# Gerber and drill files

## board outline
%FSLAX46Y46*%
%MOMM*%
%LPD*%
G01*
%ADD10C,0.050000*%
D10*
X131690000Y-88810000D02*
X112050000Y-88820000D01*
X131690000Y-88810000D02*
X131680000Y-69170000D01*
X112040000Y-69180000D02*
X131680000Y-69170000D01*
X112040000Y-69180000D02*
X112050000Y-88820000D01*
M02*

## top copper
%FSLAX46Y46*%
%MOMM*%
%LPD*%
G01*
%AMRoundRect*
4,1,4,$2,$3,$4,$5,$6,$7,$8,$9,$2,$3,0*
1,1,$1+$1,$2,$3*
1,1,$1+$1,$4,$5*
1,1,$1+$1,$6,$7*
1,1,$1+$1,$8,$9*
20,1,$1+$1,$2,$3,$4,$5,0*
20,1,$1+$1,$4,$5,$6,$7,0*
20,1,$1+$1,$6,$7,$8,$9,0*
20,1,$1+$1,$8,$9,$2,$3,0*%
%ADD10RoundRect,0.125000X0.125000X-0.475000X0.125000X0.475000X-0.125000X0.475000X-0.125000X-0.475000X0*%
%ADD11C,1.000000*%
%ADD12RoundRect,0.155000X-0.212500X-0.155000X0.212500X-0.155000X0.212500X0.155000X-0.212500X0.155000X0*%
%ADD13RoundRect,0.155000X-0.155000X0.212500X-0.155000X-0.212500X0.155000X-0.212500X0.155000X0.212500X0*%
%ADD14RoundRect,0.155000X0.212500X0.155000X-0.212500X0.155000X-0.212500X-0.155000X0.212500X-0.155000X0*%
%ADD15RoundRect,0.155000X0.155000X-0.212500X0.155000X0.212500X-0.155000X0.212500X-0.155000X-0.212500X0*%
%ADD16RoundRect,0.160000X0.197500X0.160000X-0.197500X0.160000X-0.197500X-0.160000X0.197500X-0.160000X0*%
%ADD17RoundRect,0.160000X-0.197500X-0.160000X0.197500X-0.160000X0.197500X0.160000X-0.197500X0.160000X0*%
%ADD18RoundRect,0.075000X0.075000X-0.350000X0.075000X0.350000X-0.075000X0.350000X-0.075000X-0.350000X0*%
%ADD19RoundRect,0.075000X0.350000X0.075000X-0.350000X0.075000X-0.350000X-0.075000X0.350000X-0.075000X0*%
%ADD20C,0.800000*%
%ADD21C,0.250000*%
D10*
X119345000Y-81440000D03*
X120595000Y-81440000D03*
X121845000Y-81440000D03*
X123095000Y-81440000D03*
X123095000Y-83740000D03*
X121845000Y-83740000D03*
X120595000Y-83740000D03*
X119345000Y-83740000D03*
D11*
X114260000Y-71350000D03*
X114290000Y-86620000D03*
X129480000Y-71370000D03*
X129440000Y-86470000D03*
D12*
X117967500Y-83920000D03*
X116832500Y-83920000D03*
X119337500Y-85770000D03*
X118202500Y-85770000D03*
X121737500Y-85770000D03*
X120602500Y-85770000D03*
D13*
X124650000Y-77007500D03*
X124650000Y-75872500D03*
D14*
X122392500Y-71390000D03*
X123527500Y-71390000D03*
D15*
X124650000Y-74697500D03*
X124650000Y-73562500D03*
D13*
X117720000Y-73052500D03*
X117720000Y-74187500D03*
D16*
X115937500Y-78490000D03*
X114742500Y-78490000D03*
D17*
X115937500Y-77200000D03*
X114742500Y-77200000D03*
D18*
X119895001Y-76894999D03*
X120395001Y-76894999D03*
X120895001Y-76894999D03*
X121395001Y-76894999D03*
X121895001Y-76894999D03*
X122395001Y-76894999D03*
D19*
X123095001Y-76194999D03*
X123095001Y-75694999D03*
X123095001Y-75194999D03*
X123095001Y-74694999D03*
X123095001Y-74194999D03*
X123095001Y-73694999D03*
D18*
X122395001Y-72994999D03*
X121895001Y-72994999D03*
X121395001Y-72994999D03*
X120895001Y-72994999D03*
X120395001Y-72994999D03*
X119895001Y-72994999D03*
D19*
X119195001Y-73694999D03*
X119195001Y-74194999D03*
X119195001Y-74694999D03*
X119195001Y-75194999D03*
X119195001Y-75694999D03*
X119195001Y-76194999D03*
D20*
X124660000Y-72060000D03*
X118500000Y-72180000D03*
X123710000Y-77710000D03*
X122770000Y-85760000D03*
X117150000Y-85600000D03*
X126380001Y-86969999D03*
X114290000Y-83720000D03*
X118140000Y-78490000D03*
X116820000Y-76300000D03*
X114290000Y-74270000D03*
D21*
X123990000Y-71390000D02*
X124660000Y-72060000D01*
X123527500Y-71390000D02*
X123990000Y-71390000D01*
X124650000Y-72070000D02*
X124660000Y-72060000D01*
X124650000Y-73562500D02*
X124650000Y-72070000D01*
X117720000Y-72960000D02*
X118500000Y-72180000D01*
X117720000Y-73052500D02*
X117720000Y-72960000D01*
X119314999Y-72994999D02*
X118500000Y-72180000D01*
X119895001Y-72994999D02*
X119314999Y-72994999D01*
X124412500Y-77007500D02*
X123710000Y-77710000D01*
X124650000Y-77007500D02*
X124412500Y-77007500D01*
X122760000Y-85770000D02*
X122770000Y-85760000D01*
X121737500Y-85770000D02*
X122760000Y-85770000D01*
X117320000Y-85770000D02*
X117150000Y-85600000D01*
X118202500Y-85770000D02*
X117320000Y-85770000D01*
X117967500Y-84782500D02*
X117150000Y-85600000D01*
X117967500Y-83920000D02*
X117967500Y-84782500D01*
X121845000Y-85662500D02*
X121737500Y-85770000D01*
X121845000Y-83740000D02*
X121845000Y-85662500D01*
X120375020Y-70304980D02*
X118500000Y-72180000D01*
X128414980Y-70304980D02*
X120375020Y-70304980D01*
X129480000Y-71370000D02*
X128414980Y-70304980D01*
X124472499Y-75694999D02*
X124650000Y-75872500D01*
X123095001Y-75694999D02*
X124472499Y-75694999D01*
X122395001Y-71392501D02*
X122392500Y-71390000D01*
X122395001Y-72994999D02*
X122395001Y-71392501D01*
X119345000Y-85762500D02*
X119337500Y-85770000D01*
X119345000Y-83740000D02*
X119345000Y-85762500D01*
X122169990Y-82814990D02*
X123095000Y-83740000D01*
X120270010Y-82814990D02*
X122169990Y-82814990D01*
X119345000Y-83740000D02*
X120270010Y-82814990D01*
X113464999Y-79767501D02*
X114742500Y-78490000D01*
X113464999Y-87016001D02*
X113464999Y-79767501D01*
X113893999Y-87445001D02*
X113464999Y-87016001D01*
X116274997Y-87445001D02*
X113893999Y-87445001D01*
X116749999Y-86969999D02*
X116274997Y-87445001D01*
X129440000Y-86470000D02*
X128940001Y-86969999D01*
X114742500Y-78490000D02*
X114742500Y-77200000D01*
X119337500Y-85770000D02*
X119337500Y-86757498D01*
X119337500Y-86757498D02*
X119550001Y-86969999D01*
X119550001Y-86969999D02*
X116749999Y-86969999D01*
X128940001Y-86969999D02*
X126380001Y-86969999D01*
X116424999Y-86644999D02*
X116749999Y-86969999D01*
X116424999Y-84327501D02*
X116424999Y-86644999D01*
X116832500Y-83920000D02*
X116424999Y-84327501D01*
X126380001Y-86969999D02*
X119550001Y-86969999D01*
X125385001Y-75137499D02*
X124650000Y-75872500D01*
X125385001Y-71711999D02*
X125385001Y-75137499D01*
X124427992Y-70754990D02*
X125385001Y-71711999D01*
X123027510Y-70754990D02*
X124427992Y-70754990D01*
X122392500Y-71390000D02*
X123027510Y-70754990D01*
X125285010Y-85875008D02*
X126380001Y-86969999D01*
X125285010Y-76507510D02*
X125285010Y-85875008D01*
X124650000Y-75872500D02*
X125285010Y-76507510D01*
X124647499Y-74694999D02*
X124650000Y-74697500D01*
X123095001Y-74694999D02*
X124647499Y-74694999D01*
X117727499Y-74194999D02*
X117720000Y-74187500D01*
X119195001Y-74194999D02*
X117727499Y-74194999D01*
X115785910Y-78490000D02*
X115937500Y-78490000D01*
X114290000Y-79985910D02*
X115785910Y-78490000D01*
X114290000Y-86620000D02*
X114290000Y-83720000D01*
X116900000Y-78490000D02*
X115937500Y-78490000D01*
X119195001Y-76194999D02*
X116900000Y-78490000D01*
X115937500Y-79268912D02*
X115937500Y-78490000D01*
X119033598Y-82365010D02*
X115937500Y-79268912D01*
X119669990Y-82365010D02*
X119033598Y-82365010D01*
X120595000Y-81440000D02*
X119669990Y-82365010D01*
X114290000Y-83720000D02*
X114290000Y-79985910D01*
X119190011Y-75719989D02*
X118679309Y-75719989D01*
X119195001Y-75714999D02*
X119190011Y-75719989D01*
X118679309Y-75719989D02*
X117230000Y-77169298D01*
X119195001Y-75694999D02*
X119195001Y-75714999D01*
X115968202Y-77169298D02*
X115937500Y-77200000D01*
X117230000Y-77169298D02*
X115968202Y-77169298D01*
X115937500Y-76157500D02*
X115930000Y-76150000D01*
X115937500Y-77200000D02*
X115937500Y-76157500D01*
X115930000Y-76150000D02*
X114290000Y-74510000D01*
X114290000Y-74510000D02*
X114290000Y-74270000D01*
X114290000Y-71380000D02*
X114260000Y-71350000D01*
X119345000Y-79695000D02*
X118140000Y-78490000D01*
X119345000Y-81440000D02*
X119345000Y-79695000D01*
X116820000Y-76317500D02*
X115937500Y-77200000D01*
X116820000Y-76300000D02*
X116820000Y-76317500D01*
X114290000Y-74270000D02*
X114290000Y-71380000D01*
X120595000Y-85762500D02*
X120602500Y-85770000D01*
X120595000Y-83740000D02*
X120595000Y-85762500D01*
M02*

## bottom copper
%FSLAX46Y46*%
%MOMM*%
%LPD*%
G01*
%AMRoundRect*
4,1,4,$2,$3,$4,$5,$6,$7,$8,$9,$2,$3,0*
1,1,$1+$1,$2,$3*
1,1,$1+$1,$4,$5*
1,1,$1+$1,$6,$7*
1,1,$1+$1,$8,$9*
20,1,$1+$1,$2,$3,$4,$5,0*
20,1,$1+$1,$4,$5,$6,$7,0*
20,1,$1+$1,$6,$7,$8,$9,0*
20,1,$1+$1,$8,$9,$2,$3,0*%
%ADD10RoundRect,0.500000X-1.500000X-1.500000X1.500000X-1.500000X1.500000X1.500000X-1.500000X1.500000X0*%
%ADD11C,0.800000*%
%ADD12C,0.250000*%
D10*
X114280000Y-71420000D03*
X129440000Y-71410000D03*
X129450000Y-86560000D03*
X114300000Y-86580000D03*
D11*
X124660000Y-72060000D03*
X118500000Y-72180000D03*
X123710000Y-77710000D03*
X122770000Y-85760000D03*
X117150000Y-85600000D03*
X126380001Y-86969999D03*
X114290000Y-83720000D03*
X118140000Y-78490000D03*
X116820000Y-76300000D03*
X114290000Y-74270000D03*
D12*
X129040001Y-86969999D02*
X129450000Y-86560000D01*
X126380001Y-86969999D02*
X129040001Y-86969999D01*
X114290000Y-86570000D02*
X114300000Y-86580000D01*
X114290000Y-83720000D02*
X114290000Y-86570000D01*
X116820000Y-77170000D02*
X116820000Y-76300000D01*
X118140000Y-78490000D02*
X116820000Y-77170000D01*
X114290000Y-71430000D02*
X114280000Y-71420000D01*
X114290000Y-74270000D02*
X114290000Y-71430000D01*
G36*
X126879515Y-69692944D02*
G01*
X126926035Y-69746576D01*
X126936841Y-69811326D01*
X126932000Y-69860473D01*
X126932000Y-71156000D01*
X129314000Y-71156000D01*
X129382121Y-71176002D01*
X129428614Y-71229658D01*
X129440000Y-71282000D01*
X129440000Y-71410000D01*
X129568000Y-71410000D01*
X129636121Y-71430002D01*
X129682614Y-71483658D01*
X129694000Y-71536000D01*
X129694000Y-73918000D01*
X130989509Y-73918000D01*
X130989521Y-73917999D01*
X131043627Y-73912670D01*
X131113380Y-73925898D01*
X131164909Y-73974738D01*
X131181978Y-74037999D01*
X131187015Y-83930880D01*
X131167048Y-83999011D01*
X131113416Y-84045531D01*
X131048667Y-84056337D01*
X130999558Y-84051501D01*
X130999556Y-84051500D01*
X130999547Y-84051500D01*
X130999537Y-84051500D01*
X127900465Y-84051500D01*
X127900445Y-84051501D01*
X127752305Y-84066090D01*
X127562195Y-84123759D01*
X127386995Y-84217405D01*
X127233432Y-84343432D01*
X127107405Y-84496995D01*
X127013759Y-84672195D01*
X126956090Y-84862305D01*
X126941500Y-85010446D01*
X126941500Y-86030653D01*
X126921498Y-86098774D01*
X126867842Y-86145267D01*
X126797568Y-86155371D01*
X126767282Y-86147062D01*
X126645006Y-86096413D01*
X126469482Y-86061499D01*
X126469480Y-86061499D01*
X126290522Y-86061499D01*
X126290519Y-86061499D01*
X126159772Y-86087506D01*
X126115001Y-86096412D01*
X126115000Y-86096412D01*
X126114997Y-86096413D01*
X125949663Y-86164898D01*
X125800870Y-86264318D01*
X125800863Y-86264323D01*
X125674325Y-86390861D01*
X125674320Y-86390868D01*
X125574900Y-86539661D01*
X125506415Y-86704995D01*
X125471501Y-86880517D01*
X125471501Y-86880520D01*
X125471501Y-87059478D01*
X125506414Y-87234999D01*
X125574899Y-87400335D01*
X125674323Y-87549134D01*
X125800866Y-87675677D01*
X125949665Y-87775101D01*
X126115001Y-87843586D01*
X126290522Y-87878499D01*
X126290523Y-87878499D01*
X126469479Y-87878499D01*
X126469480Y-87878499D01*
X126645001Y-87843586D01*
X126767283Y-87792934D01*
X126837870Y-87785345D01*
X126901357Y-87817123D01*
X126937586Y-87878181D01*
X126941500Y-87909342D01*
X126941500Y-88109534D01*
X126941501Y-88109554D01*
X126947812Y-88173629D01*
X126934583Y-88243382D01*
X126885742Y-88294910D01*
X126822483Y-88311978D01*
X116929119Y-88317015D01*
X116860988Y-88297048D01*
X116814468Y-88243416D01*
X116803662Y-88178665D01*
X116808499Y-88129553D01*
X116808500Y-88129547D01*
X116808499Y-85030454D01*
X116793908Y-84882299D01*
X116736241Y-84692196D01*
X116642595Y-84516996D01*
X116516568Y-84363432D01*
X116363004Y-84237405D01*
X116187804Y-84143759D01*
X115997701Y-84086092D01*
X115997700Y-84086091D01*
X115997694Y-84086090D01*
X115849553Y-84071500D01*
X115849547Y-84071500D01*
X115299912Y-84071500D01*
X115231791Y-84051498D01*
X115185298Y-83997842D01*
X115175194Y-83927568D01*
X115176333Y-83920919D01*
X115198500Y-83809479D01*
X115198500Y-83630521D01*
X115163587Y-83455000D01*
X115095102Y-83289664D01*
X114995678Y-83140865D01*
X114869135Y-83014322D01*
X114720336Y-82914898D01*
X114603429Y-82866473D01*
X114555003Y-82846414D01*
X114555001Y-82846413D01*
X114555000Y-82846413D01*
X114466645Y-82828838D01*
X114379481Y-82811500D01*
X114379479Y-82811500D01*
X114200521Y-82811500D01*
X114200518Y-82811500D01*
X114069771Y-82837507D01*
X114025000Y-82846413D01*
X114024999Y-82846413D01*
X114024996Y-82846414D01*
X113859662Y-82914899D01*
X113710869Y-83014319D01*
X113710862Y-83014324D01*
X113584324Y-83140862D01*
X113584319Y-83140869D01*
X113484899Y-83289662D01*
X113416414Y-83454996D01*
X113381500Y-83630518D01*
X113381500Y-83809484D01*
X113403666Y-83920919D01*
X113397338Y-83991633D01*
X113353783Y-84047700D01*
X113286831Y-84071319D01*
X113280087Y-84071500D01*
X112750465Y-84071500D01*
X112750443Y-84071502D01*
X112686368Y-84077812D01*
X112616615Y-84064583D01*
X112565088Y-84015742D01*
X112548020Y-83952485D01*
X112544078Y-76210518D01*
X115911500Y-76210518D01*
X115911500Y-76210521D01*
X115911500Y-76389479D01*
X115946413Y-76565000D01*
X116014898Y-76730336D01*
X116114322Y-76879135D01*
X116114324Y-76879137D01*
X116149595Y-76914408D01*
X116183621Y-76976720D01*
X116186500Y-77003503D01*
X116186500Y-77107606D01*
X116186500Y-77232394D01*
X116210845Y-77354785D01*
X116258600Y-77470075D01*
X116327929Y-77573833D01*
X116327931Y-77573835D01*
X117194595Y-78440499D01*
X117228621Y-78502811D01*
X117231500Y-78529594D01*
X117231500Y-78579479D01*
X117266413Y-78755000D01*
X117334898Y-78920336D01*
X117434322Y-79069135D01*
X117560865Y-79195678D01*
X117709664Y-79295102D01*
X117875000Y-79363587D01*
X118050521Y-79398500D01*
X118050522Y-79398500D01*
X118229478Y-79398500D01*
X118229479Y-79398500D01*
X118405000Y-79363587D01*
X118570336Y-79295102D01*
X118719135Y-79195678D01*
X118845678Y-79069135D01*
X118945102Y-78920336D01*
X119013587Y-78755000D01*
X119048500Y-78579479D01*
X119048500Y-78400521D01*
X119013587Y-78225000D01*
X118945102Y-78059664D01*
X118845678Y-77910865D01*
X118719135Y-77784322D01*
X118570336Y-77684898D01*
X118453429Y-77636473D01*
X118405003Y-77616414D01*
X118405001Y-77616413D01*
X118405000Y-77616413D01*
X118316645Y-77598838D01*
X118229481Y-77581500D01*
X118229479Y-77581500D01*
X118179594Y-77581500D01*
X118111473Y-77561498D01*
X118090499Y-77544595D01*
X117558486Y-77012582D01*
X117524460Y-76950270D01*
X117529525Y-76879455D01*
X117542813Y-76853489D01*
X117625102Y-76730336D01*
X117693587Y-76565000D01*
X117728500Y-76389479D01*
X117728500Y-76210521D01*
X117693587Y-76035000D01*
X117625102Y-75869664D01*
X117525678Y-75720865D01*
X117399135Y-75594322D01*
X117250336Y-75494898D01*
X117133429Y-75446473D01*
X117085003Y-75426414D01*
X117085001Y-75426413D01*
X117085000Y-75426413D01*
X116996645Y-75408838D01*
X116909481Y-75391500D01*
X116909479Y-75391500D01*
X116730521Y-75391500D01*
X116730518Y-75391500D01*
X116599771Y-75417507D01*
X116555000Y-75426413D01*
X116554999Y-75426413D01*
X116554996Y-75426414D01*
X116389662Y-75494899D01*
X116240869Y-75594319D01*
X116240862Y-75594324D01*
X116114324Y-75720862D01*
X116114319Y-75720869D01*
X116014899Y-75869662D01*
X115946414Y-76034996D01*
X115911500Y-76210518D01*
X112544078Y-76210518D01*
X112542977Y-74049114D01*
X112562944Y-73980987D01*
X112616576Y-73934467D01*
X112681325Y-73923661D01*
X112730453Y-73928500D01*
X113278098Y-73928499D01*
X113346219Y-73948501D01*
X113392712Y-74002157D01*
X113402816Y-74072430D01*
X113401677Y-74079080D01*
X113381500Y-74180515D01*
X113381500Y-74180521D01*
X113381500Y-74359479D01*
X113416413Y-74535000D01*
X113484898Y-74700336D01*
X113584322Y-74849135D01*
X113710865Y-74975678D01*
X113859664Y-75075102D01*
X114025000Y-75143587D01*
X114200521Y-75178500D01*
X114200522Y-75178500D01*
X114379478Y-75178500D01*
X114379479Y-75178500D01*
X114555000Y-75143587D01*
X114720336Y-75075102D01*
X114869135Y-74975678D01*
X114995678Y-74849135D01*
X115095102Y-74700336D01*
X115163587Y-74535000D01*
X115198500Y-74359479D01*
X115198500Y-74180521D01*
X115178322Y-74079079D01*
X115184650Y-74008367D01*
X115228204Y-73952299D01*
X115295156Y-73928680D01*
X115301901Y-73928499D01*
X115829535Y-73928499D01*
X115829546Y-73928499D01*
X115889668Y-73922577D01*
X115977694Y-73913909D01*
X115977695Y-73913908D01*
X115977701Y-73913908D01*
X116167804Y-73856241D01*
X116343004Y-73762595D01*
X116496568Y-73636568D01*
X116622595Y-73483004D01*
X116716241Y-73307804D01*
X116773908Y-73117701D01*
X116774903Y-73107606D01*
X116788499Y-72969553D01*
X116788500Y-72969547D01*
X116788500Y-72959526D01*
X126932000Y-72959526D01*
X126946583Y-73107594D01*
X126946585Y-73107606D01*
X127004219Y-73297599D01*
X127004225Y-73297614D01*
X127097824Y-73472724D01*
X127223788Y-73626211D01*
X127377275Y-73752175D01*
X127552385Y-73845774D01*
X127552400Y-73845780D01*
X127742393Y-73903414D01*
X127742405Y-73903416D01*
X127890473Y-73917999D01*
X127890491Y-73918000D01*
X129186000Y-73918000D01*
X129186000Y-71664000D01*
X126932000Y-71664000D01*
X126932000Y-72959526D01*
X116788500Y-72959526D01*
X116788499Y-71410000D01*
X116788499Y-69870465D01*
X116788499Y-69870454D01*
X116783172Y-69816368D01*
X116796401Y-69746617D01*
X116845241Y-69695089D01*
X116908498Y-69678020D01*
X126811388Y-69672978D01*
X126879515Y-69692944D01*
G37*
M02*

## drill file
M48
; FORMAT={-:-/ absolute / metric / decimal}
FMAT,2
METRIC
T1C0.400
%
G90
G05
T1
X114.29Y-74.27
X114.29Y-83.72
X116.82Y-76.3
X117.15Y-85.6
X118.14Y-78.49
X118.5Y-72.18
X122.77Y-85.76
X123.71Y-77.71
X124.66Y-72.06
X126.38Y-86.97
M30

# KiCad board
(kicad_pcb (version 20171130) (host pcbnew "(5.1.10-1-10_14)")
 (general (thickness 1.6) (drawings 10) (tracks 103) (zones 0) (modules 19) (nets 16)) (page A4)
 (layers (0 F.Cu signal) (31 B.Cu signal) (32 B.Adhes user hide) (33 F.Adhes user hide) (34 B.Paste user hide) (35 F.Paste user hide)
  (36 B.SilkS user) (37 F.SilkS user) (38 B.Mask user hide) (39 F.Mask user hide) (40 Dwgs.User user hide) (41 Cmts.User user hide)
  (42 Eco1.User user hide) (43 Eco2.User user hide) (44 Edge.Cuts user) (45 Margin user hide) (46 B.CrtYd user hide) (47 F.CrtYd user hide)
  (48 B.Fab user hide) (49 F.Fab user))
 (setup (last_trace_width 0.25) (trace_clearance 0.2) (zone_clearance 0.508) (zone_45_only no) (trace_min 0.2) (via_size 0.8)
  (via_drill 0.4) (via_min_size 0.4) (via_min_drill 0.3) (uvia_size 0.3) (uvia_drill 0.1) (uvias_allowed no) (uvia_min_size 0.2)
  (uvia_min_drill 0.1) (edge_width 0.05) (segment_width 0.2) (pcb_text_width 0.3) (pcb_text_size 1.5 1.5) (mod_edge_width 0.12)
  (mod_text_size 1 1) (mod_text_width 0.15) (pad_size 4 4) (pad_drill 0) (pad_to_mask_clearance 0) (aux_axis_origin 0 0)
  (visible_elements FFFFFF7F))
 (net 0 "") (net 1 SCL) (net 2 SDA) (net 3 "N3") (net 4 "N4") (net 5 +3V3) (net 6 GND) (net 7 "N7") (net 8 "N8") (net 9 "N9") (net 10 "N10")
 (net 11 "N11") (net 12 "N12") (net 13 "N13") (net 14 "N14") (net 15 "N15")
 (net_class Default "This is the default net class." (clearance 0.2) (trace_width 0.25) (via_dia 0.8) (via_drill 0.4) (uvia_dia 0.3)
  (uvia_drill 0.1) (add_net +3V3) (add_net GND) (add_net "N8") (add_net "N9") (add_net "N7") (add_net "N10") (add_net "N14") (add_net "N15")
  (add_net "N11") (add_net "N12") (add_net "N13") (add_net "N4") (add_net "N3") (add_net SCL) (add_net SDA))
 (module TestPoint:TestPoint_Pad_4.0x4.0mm (layer B.Cu) (at 114.28 71.42)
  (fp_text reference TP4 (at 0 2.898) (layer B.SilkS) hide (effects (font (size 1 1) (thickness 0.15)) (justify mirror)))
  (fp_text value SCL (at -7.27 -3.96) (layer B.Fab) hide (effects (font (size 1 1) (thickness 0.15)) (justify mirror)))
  (pad 1 smd roundrect (at 0 0) (size 4 4) (layers B.Cu B.Paste B.Mask) (roundrect_rratio 0.125) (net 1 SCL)))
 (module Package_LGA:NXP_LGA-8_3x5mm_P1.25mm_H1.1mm (layer F.Cu) (at 121.22 82.59 90)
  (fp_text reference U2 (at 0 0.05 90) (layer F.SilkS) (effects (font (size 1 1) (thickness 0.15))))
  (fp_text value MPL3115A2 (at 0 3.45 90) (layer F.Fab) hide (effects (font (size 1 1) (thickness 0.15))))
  (pad 8 smd roundrect (at 1.15 -1.875 90) (size 1.2 0.5) (layers F.Cu F.Paste F.Mask) (roundrect_rratio 0.25) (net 1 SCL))
  (pad 7 smd roundrect (at 1.15 -0.625 90) (size 1.2 0.5) (layers F.Cu F.Paste F.Mask) (roundrect_rratio 0.25) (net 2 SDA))
  (pad 6 smd roundrect (at 1.15 0.625 90) (size 1.2 0.5) (layers F.Cu F.Paste F.Mask) (roundrect_rratio 0.25) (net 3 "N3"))
  (pad 5 smd roundrect (at 1.15 1.875 90) (size 1.2 0.5) (layers F.Cu F.Paste F.Mask) (roundrect_rratio 0.25) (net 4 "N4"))
  (pad 4 smd roundrect (at -1.15 1.875 90) (size 1.2 0.5) (layers F.Cu F.Paste F.Mask) (roundrect_rratio 0.25) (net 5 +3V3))
  (pad 3 smd roundrect (at -1.15 0.625 90) (size 1.2 0.5) (layers F.Cu F.Paste F.Mask) (roundrect_rratio 0.25) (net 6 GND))
  (pad 2 smd roundrect (at -1.15 -0.625 90) (size 1.2 0.5) (layers F.Cu F.Paste F.Mask) (roundrect_rratio 0.25) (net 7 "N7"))
  (pad 1 smd roundrect (at -1.15 -1.875 90) (size 1.2 0.5) (layers F.Cu F.Paste F.Mask) (roundrect_rratio 0.25) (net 5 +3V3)))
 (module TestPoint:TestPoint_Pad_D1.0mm (layer F.Cu) (at 114.26 71.35)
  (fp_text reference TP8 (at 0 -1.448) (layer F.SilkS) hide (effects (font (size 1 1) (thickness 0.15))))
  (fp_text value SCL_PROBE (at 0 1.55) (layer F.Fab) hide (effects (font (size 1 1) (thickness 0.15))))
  (pad 1 smd circle (at 0 0) (size 1 1) (layers F.Cu F.Mask) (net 1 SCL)))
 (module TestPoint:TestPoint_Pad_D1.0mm (layer F.Cu) (at 114.29 86.62)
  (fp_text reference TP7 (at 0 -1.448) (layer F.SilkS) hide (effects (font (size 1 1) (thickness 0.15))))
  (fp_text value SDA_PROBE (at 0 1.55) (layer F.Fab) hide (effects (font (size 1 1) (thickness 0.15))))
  (pad 1 smd circle (at 0 0) (size 1 1) (layers F.Cu F.Mask) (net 2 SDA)))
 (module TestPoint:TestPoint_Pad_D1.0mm (layer F.Cu) (at 129.48 71.37)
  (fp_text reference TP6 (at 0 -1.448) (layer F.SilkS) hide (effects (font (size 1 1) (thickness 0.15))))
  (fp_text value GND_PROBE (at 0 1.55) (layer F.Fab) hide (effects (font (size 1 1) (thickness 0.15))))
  (pad 1 smd circle (at 0 0) (size 1 1) (layers F.Cu F.Mask) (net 6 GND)))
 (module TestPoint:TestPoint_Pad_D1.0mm (layer F.Cu) (at 129.44 86.47)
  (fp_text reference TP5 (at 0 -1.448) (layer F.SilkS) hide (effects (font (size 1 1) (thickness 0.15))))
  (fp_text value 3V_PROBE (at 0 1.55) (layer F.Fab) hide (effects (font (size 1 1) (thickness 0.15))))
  (pad 1 smd circle (at 0 0) (size 1 1) (layers F.Cu F.Mask) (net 5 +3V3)))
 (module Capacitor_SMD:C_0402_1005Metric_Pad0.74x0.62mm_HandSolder (layer F.Cu) (at 117.4 83.92)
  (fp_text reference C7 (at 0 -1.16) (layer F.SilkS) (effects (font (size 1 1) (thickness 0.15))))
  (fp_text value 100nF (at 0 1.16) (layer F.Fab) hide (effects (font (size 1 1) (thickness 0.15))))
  (pad 2 smd roundrect (at 0.5675 0) (size 0.735 0.62) (layers F.Cu F.Paste F.Mask) (roundrect_rratio 0.25) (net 6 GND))
  (pad 1 smd roundrect (at -0.5675 0) (size 0.735 0.62) (layers F.Cu F.Paste F.Mask) (roundrect_rratio 0.25) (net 5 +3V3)))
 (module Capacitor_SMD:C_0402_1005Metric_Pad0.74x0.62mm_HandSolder (layer F.Cu) (at 118.77 85.77)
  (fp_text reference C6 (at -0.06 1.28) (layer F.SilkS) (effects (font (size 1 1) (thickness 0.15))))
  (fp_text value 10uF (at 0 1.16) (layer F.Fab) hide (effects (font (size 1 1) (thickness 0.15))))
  (pad 2 smd roundrect (at 0.5675 0) (size 0.735 0.62) (layers F.Cu F.Paste F.Mask) (roundrect_rratio 0.25) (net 5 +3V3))
  (pad 1 smd roundrect (at -0.5675 0) (size 0.735 0.62) (layers F.Cu F.Paste F.Mask) (roundrect_rratio 0.25) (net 6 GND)))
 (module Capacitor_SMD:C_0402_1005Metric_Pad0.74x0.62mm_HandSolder (layer F.Cu) (at 121.17 85.77)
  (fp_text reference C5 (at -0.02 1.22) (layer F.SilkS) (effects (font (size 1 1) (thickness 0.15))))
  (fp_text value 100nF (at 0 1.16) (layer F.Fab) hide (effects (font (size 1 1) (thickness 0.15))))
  (pad 2 smd roundrect (at 0.5675 0) (size 0.735 0.62) (layers F.Cu F.Paste F.Mask) (roundrect_rratio 0.25) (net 6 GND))
  (pad 1 smd roundrect (at -0.5675 0) (size 0.735 0.62) (layers F.Cu F.Paste F.Mask) (roundrect_rratio 0.25) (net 7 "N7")))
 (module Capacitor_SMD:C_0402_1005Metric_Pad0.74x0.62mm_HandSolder (layer F.Cu) (at 124.65 76.44 270)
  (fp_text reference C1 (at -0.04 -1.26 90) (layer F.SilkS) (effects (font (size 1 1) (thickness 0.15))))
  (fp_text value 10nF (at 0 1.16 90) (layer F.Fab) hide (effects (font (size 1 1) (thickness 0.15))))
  (pad 2 smd roundrect (at 0.5675 0 270) (size 0.735 0.62) (layers F.Cu F.Paste F.Mask) (roundrect_rratio 0.25) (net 6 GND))
  (pad 1 smd roundrect (at -0.5675 0 270) (size 0.735 0.62) (layers F.Cu F.Paste F.Mask) (roundrect_rratio 0.25) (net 5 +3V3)))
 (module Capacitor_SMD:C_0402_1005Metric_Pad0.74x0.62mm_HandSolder (layer F.Cu) (at 122.96 71.39 180)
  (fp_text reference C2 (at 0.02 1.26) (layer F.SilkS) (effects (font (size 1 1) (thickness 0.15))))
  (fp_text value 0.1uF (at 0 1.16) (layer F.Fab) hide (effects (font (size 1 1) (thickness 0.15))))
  (pad 2 smd roundrect (at 0.5675 0 180) (size 0.735 0.62) (layers F.Cu F.Paste F.Mask) (roundrect_rratio 0.25) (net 5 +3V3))
  (pad 1 smd roundrect (at -0.5675 0 180) (size 0.735 0.62) (layers F.Cu F.Paste F.Mask) (roundrect_rratio 0.25) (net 6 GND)))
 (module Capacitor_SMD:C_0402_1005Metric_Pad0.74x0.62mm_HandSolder (layer F.Cu) (at 124.65 74.13 90)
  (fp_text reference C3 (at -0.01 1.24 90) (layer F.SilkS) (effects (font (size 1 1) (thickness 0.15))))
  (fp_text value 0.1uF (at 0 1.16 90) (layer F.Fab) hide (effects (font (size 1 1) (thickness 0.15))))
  (pad 1 smd roundrect (at -0.5675 0 90) (size 0.735 0.62) (layers F.Cu F.Paste F.Mask) (roundrect_rratio 0.25) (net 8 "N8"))
  (pad 2 smd roundrect (at 0.5675 0 90) (size 0.735 0.62) (layers F.Cu F.Paste F.Mask) (roundrect_rratio 0.25) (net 6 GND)))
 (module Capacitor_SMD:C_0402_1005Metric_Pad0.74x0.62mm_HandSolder (layer F.Cu) (at 117.72 73.62 270)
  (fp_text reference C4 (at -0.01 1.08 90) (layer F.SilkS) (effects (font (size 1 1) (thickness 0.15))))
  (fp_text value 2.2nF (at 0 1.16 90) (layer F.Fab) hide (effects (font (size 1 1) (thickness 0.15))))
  (pad 1 smd roundrect (at -0.5675 0 270) (size 0.735 0.62) (layers F.Cu F.Paste F.Mask) (roundrect_rratio 0.25) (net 6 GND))
  (pad 2 smd roundrect (at 0.5675 0 270) (size 0.735 0.62) (layers F.Cu F.Paste F.Mask) (roundrect_rratio 0.25) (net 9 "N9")))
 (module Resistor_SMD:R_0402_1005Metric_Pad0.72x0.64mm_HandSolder (layer F.Cu) (at 115.34 78.49 180)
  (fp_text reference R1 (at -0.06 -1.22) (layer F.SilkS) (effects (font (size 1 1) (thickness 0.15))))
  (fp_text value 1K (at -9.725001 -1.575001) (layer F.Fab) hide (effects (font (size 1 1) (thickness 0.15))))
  (pad 1 smd roundrect (at -0.5975 0 180) (size 0.715 0.64) (layers F.Cu F.Paste F.Mask) (roundrect_rratio 0.25) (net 2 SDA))
  (pad 2 smd roundrect (at 0.5975 0 180) (size 0.715 0.64) (layers F.Cu F.Paste F.Mask) (roundrect_rratio 0.25) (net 5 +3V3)))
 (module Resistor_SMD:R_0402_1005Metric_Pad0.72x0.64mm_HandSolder (layer F.Cu) (at 115.34 77.2)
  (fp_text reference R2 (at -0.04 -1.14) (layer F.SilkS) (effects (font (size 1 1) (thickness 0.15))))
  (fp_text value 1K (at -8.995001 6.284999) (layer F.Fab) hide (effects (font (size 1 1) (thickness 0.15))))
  (pad 2 smd roundrect (at 0.5975 0) (size 0.715 0.64) (layers F.Cu F.Paste F.Mask) (roundrect_rratio 0.25) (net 1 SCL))
  (pad 1 smd roundrect (at -0.5975 0) (size 0.715 0.64) (layers F.Cu F.Paste F.Mask) (roundrect_rratio 0.25) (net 5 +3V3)))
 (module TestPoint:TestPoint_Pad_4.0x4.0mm (layer B.Cu) (at 129.44 71.41)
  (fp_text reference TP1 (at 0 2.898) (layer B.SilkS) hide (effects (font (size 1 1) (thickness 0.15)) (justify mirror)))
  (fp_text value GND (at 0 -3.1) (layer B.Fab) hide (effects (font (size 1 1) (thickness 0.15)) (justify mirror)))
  (pad 1 smd roundrect (at 0 0) (size 4 4) (layers B.Cu B.Paste B.Mask) (roundrect_rratio 0.125) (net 6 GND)))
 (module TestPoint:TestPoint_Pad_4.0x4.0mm (layer B.Cu) (at 129.45 86.56)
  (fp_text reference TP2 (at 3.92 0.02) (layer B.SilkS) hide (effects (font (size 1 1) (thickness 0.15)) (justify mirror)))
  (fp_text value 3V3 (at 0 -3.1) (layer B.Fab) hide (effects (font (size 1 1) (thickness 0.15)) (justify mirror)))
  (pad 1 smd roundrect (at 0 0) (size 4 4) (layers B.Cu B.Paste B.Mask) (roundrect_rratio 0.125) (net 5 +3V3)))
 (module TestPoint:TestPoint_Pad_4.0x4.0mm (layer B.Cu) (at 114.3 86.58)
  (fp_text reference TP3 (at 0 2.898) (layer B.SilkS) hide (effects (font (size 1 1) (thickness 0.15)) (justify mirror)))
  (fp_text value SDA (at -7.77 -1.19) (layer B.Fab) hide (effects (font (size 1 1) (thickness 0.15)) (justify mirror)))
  (pad 1 smd roundrect (at 0 0) (size 4 4) (layers B.Cu B.Paste B.Mask) (roundrect_rratio 0.125) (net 2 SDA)))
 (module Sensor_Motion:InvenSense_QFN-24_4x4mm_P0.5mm (layer F.Cu) (at 121.145001 74.944999 90)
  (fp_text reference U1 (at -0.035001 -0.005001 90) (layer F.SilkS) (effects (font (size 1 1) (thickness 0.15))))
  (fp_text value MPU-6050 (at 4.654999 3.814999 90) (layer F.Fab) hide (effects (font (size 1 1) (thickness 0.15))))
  (pad 1 smd roundrect (at -1.95 -1.25 90) (size 0.85 0.3) (layers F.Cu F.Paste F.Mask) (roundrect_rratio 0.25) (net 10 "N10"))
  (pad 2 smd roundrect (at -1.95 -0.75 90) (size 0.85 0.3) (layers F.Cu F.Paste F.Mask) (roundrect_rratio 0.25))
  (pad 3 smd roundrect (at -1.95 -0.25 90) (size 0.85 0.3) (layers F.Cu F.Paste F.Mask) (roundrect_rratio 0.25))
  (pad 4 smd roundrect (at -1.95 0.25 90) (size 0.85 0.3) (layers F.Cu F.Paste F.Mask) (roundrect_rratio 0.25))
  (pad 5 smd roundrect (at -1.95 0.75 90) (size 0.85 0.3) (layers F.Cu F.Paste F.Mask) (roundrect_rratio 0.25))
  (pad 6 smd roundrect (at -1.95 1.25 90) (size 0.85 0.3) (layers F.Cu F.Paste F.Mask) (roundrect_rratio 0.25) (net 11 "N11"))
  (pad 7 smd roundrect (at -1.25 1.95 180) (size 0.85 0.3) (layers F.Cu F.Paste F.Mask) (roundrect_rratio 0.25) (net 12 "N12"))
  (pad 8 smd roundrect (at -0.75 1.95 180) (size 0.85 0.3) (layers F.Cu F.Paste F.Mask) (roundrect_rratio 0.25) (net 5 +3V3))
  (pad 9 smd roundrect (at -0.25 1.95 180) (size 0.85 0.3) (layers F.Cu F.Paste F.Mask) (roundrect_rratio 0.25) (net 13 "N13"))
  (pad 10 smd roundrect (at 0.25 1.95 180) (size 0.85 0.3) (layers F.Cu F.Paste F.Mask) (roundrect_rratio 0.25) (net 8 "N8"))
  (pad 11 smd roundrect (at 0.75 1.95 180) (size 0.85 0.3) (layers F.Cu F.Paste F.Mask) (roundrect_rratio 0.25) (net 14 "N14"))
  (pad 12 smd roundrect (at 1.25 1.95 180) (size 0.85 0.3) (layers F.Cu F.Paste F.Mask) (roundrect_rratio 0.25) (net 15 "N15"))
  (pad 13 smd roundrect (at 1.95 1.25 90) (size 0.85 0.3) (layers F.Cu F.Paste F.Mask) (roundrect_rratio 0.25) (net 5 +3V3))
  (pad 14 smd roundrect (at 1.95 0.75 90) (size 0.85 0.3) (layers F.Cu F.Paste F.Mask) (roundrect_rratio 0.25))
  (pad 15 smd roundrect (at 1.95 0.25 90) (size 0.85 0.3) (layers F.Cu F.Paste F.Mask) (roundrect_rratio 0.25))
  (pad 16 smd roundrect (at 1.95 -0.25 90) (size 0.85 0.3) (layers F.Cu F.Paste F.Mask) (roundrect_rratio 0.25))
  (pad 17 smd roundrect (at 1.95 -0.75 90) (size 0.85 0.3) (layers F.Cu F.Paste F.Mask) (roundrect_rratio 0.25))
  (pad 18 smd roundrect (at 1.95 -1.25 90) (size 0.85 0.3) (layers F.Cu F.Paste F.Mask) (roundrect_rratio 0.25) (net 6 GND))
  (pad 19 smd roundrect (at 1.25 -1.95 180) (size 0.85 0.3) (layers F.Cu F.Paste F.Mask) (roundrect_rratio 0.25))
  (pad 20 smd roundrect (at 0.75 -1.95 180) (size 0.85 0.3) (layers F.Cu F.Paste F.Mask) (roundrect_rratio 0.25) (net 9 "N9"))
  (pad 21 smd roundrect (at 0.25 -1.95 180) (size 0.85 0.3) (layers F.Cu F.Paste F.Mask) (roundrect_rratio 0.25))
  (pad 22 smd roundrect (at -0.25 -1.95 180) (size 0.85 0.3) (layers F.Cu F.Paste F.Mask) (roundrect_rratio 0.25))
  (pad 23 smd roundrect (at -0.75 -1.95 180) (size 0.85 0.3) (layers F.Cu F.Paste F.Mask) (roundrect_rratio 0.25) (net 1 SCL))
  (pad 24 smd roundrect (at -1.25 -1.95 180) (size 0.85 0.3) (layers F.Cu F.Paste F.Mask) (roundrect_rratio 0.25) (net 2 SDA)))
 (gr_line (start 131.69 88.81) (end 112.05 88.82) (layer Edge.Cuts) (width 0.05))
 (gr_line (start 131.69 88.81) (end 131.68 69.17) (layer Edge.Cuts) (width 0.05))
 (gr_line (start 112.04 69.18) (end 131.68 69.17) (layer Edge.Cuts) (width 0.05))
 (gr_line (start 112.04 69.18) (end 112.05 88.82) (layer Edge.Cuts) (width 0.05))
 (via (at 124.66 72.06) (size 0.8) (drill 0.4) (layers F.Cu B.Cu) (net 6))
 (segment (start 123.99 71.39) (end 124.66 72.06) (width 0.25) (layer F.Cu) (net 6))
 (segment (start 123.5275 71.39) (end 123.99 71.39) (width 0.25) (layer F.Cu) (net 6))
 (segment (start 124.65 72.07) (end 124.66 72.06) (width 0.25) (layer F.Cu) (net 6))
 (segment (start 124.65 73.5625) (end 124.65 72.07) (width 0.25) (layer F.Cu) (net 6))
 (via (at 118.5 72.18) (size 0.8) (drill 0.4) (layers F.Cu B.Cu) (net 6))
 (segment (start 117.72 72.96) (end 118.5 72.18) (width 0.25) (layer F.Cu) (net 6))
 (segment (start 117.72 73.0525) (end 117.72 72.96) (width 0.25) (layer F.Cu) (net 6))
 (segment (start 119.314999 72.994999) (end 118.5 72.18) (width 0.25) (layer F.Cu) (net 6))
 (segment (start 119.895001 72.994999) (end 119.314999 72.994999) (width 0.25) (layer F.Cu) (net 6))
 (via (at 123.71 77.71) (size 0.8) (drill 0.4) (layers F.Cu B.Cu) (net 6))
 (segment (start 124.4125 77.0075) (end 123.71 77.71) (width 0.25) (layer F.Cu) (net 6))
 (segment (start 124.65 77.0075) (end 124.4125 77.0075) (width 0.25) (layer F.Cu) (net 6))
 (via (at 122.77 85.76) (size 0.8) (drill 0.4) (layers F.Cu B.Cu) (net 6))
 (segment (start 122.76 85.77) (end 122.77 85.76) (width 0.25) (layer F.Cu) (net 6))
 (segment (start 121.7375 85.77) (end 122.76 85.77) (width 0.25) (layer F.Cu) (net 6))
 (via (at 117.15 85.6) (size 0.8) (drill 0.4) (layers F.Cu B.Cu) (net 6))
 (segment (start 117.32 85.77) (end 117.15 85.6) (width 0.25) (layer F.Cu) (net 6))
 (segment (start 118.2025 85.77) (end 117.32 85.77) (width 0.25) (layer F.Cu) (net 6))
 (segment (start 117.9675 84.7825) (end 117.15 85.6) (width 0.25) (layer F.Cu) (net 6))
 (segment (start 117.9675 83.92) (end 117.9675 84.7825) (width 0.25) (layer F.Cu) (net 6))
 (segment (start 121.845 85.6625) (end 121.7375 85.77) (width 0.25) (layer F.Cu) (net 6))
 (segment (start 121.845 83.74) (end 121.845 85.6625) (width 0.25) (layer F.Cu) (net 6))
 (segment (start 120.37502 70.30498) (end 118.5 72.18) (width 0.25) (layer F.Cu) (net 6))
 (segment (start 128.41498 70.30498) (end 120.37502 70.30498) (width 0.25) (layer F.Cu) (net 6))
 (segment (start 129.48 71.37) (end 128.41498 70.30498) (width 0.25) (layer F.Cu) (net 6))
 (segment (start 124.472499 75.694999) (end 124.65 75.8725) (width 0.25) (layer F.Cu) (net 5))
 (segment (start 123.095001 75.694999) (end 124.472499 75.694999) (width 0.25) (layer F.Cu) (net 5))
 (segment (start 122.395001 71.392501) (end 122.3925 71.39) (width 0.25) (layer F.Cu) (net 5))
 (segment (start 122.395001 72.994999) (end 122.395001 71.392501) (width 0.25) (layer F.Cu) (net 5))
 (segment (start 119.345 85.7625) (end 119.3375 85.77) (width 0.25) (layer F.Cu) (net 5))
 (segment (start 119.345 83.74) (end 119.345 85.7625) (width 0.25) (layer F.Cu) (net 5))
 (segment (start 122.16999 82.81499) (end 123.095 83.74) (width 0.25) (layer F.Cu) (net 5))
 (segment (start 120.27001 82.81499) (end 122.16999 82.81499) (width 0.25) (layer F.Cu) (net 5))
 (segment (start 119.345 83.74) (end 120.27001 82.81499) (width 0.25) (layer F.Cu) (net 5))
 (segment (start 113.464999 79.767501) (end 114.7425 78.49) (width 0.25) (layer F.Cu) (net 5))
 (segment (start 113.464999 87.016001) (end 113.464999 79.767501) (width 0.25) (layer F.Cu) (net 5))
 (segment (start 113.893999 87.445001) (end 113.464999 87.016001) (width 0.25) (layer F.Cu) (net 5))
 (segment (start 116.274997 87.445001) (end 113.893999 87.445001) (width 0.25) (layer F.Cu) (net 5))
 (segment (start 116.749999 86.969999) (end 116.274997 87.445001) (width 0.25) (layer F.Cu) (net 5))
 (segment (start 129.44 86.47) (end 128.940001 86.969999) (width 0.25) (layer F.Cu) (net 5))
 (segment (start 114.7425 78.49) (end 114.7425 77.2) (width 0.25) (layer F.Cu) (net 5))
 (segment (start 119.3375 85.77) (end 119.3375 86.757498) (width 0.25) (layer F.Cu) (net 5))
 (segment (start 119.3375 86.757498) (end 119.550001 86.969999) (width 0.25) (layer F.Cu) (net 5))
 (segment (start 119.550001 86.969999) (end 116.749999 86.969999) (width 0.25) (layer F.Cu) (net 5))
 (segment (start 128.940001 86.969999) (end 126.380001 86.969999) (width 0.25) (layer F.Cu) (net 5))
 (segment (start 116.424999 86.644999) (end 116.749999 86.969999) (width 0.25) (layer F.Cu) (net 5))
 (segment (start 116.424999 84.327501) (end 116.424999 86.644999) (width 0.25) (layer F.Cu) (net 5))
 (segment (start 116.8325 83.92) (end 116.424999 84.327501) (width 0.25) (layer F.Cu) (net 5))
 (segment (start 126.380001 86.969999) (end 119.550001 86.969999) (width 0.25) (layer F.Cu) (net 5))
 (via (at 126.380001 86.969999) (size 0.8) (drill 0.4) (layers F.Cu B.Cu) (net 5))
 (segment (start 129.040001 86.969999) (end 129.45 86.56) (width 0.25) (layer B.Cu) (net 5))
 (segment (start 126.380001 86.969999) (end 129.040001 86.969999) (width 0.25) (layer B.Cu) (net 5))
 (segment (start 125.385001 75.137499) (end 124.65 75.8725) (width 0.25) (layer F.Cu) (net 5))
 (segment (start 125.385001 71.711999) (end 125.385001 75.137499) (width 0.25) (layer F.Cu) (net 5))
 (segment (start 124.427992 70.75499) (end 125.385001 71.711999) (width 0.25) (layer F.Cu) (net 5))
 (segment (start 123.02751 70.75499) (end 124.427992 70.75499) (width 0.25) (layer F.Cu) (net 5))
 (segment (start 122.3925 71.39) (end 123.02751 70.75499) (width 0.25) (layer F.Cu) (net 5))
 (segment (start 125.28501 85.875008) (end 126.380001 86.969999) (width 0.25) (layer F.Cu) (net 5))
 (segment (start 125.28501 76.50751) (end 125.28501 85.875008) (width 0.25) (layer F.Cu) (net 5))
 (segment (start 124.65 75.8725) (end 125.28501 76.50751) (width 0.25) (layer F.Cu) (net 5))
 (segment (start 124.647499 74.694999) (end 124.65 74.6975) (width 0.25) (layer F.Cu) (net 8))
 (segment (start 123.095001 74.694999) (end 124.647499 74.694999) (width 0.25) (layer F.Cu) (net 8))
 (segment (start 117.727499 74.194999) (end 117.72 74.1875) (width 0.25) (layer F.Cu) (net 9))
 (segment (start 119.195001 74.194999) (end 117.727499 74.194999) (width 0.25) (layer F.Cu) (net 9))
 (segment (start 115.78591 78.49) (end 115.9375 78.49) (width 0.25) (layer F.Cu) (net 2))
 (segment (start 114.29 79.98591) (end 115.78591 78.49) (width 0.25) (layer F.Cu) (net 2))
 (segment (start 114.29 86.62) (end 114.29 83.72) (width 0.25) (layer F.Cu) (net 2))
 (segment (start 116.9 78.49) (end 115.9375 78.49) (width 0.25) (layer F.Cu) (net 2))
 (segment (start 119.195001 76.194999) (end 116.9 78.49) (width 0.25) (layer F.Cu) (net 2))
 (segment (start 115.9375 79.268912) (end 115.9375 78.49) (width 0.25) (layer F.Cu) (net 2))
 (segment (start 119.033598 82.36501) (end 115.9375 79.268912) (width 0.25) (layer F.Cu) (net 2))
 (segment (start 119.66999 82.36501) (end 119.033598 82.36501) (width 0.25) (layer F.Cu) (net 2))
 (segment (start 120.595 81.44) (end 119.66999 82.36501) (width 0.25) (layer F.Cu) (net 2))
 (segment (start 114.29 83.72) (end 114.29 79.98591) (width 0.25) (layer F.Cu) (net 2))
 (via (at 114.29 83.72) (size 0.8) (drill 0.4) (layers F.Cu B.Cu) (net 2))
 (segment (start 114.29 86.57) (end 114.3 86.58) (width 0.25) (layer B.Cu) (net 2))
 (segment (start 114.29 83.72) (end 114.29 86.57) (width 0.25) (layer B.Cu) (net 2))
 (segment (start 119.190011 75.719989) (end 118.679309 75.719989) (width 0.25) (layer F.Cu) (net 1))
 (segment (start 119.195001 75.714999) (end 119.190011 75.719989) (width 0.25) (layer F.Cu) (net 1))
 (segment (start 118.679309 75.719989) (end 117.23 77.169298) (width 0.25) (layer F.Cu) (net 1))
 (segment (start 119.195001 75.694999) (end 119.195001 75.714999) (width 0.25) (layer F.Cu) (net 1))
 (segment (start 115.968202 77.169298) (end 115.9375 77.2) (width 0.25) (layer F.Cu) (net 1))
 (segment (start 117.23 77.169298) (end 115.968202 77.169298) (width 0.25) (layer F.Cu) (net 1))
 (segment (start 115.9375 76.1575) (end 115.93 76.15) (width 0.25) (layer F.Cu) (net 1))
 (segment (start 115.9375 77.2) (end 115.9375 76.1575) (width 0.25) (layer F.Cu) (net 1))
 (segment (start 115.93 76.15) (end 114.29 74.51) (width 0.25) (layer F.Cu) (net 1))
 (segment (start 114.29 74.51) (end 114.29 74.27) (width 0.25) (layer F.Cu) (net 1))
 (segment (start 114.29 71.38) (end 114.26 71.35) (width 0.25) (layer F.Cu) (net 1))
 (via (at 118.14 78.49) (size 0.8) (drill 0.4) (layers F.Cu B.Cu) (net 1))
 (segment (start 119.345 79.695) (end 118.14 78.49) (width 0.25) (layer F.Cu) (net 1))
 (segment (start 119.345 81.44) (end 119.345 79.695) (width 0.25) (layer F.Cu) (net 1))
 (via (at 116.82 76.3) (size 0.8) (drill 0.4) (layers F.Cu B.Cu) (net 1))
 (segment (start 116.82 77.17) (end 116.82 76.3) (width 0.25) (layer B.Cu) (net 1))
 (segment (start 118.14 78.49) (end 116.82 77.17) (width 0.25) (layer B.Cu) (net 1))
 (segment (start 116.82 76.3175) (end 115.9375 77.2) (width 0.25) (layer F.Cu) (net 1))
 (segment (start 116.82 76.3) (end 116.82 76.3175) (width 0.25) (layer F.Cu) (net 1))
 (segment (start 114.29 74.27) (end 114.29 71.38) (width 0.25) (layer F.Cu) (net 1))
 (via (at 114.29 74.27) (size 0.8) (drill 0.4) (layers F.Cu B.Cu) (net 1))
 (segment (start 114.29 71.43) (end 114.28 71.42) (width 0.25) (layer B.Cu) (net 1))
 (segment (start 114.29 74.27) (end 114.29 71.43) (width 0.25) (layer B.Cu) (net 1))
 (segment (start 120.595 85.7625) (end 120.6025 85.77) (width 0.25) (layer F.Cu) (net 7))
 (segment (start 120.595 83.74) (end 120.595 85.7625) (width 0.25) (layer F.Cu) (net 7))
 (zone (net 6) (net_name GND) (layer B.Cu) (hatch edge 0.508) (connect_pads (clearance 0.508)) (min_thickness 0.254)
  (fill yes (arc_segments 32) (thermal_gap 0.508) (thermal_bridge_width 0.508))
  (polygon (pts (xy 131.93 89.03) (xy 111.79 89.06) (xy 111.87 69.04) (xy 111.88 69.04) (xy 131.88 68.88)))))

